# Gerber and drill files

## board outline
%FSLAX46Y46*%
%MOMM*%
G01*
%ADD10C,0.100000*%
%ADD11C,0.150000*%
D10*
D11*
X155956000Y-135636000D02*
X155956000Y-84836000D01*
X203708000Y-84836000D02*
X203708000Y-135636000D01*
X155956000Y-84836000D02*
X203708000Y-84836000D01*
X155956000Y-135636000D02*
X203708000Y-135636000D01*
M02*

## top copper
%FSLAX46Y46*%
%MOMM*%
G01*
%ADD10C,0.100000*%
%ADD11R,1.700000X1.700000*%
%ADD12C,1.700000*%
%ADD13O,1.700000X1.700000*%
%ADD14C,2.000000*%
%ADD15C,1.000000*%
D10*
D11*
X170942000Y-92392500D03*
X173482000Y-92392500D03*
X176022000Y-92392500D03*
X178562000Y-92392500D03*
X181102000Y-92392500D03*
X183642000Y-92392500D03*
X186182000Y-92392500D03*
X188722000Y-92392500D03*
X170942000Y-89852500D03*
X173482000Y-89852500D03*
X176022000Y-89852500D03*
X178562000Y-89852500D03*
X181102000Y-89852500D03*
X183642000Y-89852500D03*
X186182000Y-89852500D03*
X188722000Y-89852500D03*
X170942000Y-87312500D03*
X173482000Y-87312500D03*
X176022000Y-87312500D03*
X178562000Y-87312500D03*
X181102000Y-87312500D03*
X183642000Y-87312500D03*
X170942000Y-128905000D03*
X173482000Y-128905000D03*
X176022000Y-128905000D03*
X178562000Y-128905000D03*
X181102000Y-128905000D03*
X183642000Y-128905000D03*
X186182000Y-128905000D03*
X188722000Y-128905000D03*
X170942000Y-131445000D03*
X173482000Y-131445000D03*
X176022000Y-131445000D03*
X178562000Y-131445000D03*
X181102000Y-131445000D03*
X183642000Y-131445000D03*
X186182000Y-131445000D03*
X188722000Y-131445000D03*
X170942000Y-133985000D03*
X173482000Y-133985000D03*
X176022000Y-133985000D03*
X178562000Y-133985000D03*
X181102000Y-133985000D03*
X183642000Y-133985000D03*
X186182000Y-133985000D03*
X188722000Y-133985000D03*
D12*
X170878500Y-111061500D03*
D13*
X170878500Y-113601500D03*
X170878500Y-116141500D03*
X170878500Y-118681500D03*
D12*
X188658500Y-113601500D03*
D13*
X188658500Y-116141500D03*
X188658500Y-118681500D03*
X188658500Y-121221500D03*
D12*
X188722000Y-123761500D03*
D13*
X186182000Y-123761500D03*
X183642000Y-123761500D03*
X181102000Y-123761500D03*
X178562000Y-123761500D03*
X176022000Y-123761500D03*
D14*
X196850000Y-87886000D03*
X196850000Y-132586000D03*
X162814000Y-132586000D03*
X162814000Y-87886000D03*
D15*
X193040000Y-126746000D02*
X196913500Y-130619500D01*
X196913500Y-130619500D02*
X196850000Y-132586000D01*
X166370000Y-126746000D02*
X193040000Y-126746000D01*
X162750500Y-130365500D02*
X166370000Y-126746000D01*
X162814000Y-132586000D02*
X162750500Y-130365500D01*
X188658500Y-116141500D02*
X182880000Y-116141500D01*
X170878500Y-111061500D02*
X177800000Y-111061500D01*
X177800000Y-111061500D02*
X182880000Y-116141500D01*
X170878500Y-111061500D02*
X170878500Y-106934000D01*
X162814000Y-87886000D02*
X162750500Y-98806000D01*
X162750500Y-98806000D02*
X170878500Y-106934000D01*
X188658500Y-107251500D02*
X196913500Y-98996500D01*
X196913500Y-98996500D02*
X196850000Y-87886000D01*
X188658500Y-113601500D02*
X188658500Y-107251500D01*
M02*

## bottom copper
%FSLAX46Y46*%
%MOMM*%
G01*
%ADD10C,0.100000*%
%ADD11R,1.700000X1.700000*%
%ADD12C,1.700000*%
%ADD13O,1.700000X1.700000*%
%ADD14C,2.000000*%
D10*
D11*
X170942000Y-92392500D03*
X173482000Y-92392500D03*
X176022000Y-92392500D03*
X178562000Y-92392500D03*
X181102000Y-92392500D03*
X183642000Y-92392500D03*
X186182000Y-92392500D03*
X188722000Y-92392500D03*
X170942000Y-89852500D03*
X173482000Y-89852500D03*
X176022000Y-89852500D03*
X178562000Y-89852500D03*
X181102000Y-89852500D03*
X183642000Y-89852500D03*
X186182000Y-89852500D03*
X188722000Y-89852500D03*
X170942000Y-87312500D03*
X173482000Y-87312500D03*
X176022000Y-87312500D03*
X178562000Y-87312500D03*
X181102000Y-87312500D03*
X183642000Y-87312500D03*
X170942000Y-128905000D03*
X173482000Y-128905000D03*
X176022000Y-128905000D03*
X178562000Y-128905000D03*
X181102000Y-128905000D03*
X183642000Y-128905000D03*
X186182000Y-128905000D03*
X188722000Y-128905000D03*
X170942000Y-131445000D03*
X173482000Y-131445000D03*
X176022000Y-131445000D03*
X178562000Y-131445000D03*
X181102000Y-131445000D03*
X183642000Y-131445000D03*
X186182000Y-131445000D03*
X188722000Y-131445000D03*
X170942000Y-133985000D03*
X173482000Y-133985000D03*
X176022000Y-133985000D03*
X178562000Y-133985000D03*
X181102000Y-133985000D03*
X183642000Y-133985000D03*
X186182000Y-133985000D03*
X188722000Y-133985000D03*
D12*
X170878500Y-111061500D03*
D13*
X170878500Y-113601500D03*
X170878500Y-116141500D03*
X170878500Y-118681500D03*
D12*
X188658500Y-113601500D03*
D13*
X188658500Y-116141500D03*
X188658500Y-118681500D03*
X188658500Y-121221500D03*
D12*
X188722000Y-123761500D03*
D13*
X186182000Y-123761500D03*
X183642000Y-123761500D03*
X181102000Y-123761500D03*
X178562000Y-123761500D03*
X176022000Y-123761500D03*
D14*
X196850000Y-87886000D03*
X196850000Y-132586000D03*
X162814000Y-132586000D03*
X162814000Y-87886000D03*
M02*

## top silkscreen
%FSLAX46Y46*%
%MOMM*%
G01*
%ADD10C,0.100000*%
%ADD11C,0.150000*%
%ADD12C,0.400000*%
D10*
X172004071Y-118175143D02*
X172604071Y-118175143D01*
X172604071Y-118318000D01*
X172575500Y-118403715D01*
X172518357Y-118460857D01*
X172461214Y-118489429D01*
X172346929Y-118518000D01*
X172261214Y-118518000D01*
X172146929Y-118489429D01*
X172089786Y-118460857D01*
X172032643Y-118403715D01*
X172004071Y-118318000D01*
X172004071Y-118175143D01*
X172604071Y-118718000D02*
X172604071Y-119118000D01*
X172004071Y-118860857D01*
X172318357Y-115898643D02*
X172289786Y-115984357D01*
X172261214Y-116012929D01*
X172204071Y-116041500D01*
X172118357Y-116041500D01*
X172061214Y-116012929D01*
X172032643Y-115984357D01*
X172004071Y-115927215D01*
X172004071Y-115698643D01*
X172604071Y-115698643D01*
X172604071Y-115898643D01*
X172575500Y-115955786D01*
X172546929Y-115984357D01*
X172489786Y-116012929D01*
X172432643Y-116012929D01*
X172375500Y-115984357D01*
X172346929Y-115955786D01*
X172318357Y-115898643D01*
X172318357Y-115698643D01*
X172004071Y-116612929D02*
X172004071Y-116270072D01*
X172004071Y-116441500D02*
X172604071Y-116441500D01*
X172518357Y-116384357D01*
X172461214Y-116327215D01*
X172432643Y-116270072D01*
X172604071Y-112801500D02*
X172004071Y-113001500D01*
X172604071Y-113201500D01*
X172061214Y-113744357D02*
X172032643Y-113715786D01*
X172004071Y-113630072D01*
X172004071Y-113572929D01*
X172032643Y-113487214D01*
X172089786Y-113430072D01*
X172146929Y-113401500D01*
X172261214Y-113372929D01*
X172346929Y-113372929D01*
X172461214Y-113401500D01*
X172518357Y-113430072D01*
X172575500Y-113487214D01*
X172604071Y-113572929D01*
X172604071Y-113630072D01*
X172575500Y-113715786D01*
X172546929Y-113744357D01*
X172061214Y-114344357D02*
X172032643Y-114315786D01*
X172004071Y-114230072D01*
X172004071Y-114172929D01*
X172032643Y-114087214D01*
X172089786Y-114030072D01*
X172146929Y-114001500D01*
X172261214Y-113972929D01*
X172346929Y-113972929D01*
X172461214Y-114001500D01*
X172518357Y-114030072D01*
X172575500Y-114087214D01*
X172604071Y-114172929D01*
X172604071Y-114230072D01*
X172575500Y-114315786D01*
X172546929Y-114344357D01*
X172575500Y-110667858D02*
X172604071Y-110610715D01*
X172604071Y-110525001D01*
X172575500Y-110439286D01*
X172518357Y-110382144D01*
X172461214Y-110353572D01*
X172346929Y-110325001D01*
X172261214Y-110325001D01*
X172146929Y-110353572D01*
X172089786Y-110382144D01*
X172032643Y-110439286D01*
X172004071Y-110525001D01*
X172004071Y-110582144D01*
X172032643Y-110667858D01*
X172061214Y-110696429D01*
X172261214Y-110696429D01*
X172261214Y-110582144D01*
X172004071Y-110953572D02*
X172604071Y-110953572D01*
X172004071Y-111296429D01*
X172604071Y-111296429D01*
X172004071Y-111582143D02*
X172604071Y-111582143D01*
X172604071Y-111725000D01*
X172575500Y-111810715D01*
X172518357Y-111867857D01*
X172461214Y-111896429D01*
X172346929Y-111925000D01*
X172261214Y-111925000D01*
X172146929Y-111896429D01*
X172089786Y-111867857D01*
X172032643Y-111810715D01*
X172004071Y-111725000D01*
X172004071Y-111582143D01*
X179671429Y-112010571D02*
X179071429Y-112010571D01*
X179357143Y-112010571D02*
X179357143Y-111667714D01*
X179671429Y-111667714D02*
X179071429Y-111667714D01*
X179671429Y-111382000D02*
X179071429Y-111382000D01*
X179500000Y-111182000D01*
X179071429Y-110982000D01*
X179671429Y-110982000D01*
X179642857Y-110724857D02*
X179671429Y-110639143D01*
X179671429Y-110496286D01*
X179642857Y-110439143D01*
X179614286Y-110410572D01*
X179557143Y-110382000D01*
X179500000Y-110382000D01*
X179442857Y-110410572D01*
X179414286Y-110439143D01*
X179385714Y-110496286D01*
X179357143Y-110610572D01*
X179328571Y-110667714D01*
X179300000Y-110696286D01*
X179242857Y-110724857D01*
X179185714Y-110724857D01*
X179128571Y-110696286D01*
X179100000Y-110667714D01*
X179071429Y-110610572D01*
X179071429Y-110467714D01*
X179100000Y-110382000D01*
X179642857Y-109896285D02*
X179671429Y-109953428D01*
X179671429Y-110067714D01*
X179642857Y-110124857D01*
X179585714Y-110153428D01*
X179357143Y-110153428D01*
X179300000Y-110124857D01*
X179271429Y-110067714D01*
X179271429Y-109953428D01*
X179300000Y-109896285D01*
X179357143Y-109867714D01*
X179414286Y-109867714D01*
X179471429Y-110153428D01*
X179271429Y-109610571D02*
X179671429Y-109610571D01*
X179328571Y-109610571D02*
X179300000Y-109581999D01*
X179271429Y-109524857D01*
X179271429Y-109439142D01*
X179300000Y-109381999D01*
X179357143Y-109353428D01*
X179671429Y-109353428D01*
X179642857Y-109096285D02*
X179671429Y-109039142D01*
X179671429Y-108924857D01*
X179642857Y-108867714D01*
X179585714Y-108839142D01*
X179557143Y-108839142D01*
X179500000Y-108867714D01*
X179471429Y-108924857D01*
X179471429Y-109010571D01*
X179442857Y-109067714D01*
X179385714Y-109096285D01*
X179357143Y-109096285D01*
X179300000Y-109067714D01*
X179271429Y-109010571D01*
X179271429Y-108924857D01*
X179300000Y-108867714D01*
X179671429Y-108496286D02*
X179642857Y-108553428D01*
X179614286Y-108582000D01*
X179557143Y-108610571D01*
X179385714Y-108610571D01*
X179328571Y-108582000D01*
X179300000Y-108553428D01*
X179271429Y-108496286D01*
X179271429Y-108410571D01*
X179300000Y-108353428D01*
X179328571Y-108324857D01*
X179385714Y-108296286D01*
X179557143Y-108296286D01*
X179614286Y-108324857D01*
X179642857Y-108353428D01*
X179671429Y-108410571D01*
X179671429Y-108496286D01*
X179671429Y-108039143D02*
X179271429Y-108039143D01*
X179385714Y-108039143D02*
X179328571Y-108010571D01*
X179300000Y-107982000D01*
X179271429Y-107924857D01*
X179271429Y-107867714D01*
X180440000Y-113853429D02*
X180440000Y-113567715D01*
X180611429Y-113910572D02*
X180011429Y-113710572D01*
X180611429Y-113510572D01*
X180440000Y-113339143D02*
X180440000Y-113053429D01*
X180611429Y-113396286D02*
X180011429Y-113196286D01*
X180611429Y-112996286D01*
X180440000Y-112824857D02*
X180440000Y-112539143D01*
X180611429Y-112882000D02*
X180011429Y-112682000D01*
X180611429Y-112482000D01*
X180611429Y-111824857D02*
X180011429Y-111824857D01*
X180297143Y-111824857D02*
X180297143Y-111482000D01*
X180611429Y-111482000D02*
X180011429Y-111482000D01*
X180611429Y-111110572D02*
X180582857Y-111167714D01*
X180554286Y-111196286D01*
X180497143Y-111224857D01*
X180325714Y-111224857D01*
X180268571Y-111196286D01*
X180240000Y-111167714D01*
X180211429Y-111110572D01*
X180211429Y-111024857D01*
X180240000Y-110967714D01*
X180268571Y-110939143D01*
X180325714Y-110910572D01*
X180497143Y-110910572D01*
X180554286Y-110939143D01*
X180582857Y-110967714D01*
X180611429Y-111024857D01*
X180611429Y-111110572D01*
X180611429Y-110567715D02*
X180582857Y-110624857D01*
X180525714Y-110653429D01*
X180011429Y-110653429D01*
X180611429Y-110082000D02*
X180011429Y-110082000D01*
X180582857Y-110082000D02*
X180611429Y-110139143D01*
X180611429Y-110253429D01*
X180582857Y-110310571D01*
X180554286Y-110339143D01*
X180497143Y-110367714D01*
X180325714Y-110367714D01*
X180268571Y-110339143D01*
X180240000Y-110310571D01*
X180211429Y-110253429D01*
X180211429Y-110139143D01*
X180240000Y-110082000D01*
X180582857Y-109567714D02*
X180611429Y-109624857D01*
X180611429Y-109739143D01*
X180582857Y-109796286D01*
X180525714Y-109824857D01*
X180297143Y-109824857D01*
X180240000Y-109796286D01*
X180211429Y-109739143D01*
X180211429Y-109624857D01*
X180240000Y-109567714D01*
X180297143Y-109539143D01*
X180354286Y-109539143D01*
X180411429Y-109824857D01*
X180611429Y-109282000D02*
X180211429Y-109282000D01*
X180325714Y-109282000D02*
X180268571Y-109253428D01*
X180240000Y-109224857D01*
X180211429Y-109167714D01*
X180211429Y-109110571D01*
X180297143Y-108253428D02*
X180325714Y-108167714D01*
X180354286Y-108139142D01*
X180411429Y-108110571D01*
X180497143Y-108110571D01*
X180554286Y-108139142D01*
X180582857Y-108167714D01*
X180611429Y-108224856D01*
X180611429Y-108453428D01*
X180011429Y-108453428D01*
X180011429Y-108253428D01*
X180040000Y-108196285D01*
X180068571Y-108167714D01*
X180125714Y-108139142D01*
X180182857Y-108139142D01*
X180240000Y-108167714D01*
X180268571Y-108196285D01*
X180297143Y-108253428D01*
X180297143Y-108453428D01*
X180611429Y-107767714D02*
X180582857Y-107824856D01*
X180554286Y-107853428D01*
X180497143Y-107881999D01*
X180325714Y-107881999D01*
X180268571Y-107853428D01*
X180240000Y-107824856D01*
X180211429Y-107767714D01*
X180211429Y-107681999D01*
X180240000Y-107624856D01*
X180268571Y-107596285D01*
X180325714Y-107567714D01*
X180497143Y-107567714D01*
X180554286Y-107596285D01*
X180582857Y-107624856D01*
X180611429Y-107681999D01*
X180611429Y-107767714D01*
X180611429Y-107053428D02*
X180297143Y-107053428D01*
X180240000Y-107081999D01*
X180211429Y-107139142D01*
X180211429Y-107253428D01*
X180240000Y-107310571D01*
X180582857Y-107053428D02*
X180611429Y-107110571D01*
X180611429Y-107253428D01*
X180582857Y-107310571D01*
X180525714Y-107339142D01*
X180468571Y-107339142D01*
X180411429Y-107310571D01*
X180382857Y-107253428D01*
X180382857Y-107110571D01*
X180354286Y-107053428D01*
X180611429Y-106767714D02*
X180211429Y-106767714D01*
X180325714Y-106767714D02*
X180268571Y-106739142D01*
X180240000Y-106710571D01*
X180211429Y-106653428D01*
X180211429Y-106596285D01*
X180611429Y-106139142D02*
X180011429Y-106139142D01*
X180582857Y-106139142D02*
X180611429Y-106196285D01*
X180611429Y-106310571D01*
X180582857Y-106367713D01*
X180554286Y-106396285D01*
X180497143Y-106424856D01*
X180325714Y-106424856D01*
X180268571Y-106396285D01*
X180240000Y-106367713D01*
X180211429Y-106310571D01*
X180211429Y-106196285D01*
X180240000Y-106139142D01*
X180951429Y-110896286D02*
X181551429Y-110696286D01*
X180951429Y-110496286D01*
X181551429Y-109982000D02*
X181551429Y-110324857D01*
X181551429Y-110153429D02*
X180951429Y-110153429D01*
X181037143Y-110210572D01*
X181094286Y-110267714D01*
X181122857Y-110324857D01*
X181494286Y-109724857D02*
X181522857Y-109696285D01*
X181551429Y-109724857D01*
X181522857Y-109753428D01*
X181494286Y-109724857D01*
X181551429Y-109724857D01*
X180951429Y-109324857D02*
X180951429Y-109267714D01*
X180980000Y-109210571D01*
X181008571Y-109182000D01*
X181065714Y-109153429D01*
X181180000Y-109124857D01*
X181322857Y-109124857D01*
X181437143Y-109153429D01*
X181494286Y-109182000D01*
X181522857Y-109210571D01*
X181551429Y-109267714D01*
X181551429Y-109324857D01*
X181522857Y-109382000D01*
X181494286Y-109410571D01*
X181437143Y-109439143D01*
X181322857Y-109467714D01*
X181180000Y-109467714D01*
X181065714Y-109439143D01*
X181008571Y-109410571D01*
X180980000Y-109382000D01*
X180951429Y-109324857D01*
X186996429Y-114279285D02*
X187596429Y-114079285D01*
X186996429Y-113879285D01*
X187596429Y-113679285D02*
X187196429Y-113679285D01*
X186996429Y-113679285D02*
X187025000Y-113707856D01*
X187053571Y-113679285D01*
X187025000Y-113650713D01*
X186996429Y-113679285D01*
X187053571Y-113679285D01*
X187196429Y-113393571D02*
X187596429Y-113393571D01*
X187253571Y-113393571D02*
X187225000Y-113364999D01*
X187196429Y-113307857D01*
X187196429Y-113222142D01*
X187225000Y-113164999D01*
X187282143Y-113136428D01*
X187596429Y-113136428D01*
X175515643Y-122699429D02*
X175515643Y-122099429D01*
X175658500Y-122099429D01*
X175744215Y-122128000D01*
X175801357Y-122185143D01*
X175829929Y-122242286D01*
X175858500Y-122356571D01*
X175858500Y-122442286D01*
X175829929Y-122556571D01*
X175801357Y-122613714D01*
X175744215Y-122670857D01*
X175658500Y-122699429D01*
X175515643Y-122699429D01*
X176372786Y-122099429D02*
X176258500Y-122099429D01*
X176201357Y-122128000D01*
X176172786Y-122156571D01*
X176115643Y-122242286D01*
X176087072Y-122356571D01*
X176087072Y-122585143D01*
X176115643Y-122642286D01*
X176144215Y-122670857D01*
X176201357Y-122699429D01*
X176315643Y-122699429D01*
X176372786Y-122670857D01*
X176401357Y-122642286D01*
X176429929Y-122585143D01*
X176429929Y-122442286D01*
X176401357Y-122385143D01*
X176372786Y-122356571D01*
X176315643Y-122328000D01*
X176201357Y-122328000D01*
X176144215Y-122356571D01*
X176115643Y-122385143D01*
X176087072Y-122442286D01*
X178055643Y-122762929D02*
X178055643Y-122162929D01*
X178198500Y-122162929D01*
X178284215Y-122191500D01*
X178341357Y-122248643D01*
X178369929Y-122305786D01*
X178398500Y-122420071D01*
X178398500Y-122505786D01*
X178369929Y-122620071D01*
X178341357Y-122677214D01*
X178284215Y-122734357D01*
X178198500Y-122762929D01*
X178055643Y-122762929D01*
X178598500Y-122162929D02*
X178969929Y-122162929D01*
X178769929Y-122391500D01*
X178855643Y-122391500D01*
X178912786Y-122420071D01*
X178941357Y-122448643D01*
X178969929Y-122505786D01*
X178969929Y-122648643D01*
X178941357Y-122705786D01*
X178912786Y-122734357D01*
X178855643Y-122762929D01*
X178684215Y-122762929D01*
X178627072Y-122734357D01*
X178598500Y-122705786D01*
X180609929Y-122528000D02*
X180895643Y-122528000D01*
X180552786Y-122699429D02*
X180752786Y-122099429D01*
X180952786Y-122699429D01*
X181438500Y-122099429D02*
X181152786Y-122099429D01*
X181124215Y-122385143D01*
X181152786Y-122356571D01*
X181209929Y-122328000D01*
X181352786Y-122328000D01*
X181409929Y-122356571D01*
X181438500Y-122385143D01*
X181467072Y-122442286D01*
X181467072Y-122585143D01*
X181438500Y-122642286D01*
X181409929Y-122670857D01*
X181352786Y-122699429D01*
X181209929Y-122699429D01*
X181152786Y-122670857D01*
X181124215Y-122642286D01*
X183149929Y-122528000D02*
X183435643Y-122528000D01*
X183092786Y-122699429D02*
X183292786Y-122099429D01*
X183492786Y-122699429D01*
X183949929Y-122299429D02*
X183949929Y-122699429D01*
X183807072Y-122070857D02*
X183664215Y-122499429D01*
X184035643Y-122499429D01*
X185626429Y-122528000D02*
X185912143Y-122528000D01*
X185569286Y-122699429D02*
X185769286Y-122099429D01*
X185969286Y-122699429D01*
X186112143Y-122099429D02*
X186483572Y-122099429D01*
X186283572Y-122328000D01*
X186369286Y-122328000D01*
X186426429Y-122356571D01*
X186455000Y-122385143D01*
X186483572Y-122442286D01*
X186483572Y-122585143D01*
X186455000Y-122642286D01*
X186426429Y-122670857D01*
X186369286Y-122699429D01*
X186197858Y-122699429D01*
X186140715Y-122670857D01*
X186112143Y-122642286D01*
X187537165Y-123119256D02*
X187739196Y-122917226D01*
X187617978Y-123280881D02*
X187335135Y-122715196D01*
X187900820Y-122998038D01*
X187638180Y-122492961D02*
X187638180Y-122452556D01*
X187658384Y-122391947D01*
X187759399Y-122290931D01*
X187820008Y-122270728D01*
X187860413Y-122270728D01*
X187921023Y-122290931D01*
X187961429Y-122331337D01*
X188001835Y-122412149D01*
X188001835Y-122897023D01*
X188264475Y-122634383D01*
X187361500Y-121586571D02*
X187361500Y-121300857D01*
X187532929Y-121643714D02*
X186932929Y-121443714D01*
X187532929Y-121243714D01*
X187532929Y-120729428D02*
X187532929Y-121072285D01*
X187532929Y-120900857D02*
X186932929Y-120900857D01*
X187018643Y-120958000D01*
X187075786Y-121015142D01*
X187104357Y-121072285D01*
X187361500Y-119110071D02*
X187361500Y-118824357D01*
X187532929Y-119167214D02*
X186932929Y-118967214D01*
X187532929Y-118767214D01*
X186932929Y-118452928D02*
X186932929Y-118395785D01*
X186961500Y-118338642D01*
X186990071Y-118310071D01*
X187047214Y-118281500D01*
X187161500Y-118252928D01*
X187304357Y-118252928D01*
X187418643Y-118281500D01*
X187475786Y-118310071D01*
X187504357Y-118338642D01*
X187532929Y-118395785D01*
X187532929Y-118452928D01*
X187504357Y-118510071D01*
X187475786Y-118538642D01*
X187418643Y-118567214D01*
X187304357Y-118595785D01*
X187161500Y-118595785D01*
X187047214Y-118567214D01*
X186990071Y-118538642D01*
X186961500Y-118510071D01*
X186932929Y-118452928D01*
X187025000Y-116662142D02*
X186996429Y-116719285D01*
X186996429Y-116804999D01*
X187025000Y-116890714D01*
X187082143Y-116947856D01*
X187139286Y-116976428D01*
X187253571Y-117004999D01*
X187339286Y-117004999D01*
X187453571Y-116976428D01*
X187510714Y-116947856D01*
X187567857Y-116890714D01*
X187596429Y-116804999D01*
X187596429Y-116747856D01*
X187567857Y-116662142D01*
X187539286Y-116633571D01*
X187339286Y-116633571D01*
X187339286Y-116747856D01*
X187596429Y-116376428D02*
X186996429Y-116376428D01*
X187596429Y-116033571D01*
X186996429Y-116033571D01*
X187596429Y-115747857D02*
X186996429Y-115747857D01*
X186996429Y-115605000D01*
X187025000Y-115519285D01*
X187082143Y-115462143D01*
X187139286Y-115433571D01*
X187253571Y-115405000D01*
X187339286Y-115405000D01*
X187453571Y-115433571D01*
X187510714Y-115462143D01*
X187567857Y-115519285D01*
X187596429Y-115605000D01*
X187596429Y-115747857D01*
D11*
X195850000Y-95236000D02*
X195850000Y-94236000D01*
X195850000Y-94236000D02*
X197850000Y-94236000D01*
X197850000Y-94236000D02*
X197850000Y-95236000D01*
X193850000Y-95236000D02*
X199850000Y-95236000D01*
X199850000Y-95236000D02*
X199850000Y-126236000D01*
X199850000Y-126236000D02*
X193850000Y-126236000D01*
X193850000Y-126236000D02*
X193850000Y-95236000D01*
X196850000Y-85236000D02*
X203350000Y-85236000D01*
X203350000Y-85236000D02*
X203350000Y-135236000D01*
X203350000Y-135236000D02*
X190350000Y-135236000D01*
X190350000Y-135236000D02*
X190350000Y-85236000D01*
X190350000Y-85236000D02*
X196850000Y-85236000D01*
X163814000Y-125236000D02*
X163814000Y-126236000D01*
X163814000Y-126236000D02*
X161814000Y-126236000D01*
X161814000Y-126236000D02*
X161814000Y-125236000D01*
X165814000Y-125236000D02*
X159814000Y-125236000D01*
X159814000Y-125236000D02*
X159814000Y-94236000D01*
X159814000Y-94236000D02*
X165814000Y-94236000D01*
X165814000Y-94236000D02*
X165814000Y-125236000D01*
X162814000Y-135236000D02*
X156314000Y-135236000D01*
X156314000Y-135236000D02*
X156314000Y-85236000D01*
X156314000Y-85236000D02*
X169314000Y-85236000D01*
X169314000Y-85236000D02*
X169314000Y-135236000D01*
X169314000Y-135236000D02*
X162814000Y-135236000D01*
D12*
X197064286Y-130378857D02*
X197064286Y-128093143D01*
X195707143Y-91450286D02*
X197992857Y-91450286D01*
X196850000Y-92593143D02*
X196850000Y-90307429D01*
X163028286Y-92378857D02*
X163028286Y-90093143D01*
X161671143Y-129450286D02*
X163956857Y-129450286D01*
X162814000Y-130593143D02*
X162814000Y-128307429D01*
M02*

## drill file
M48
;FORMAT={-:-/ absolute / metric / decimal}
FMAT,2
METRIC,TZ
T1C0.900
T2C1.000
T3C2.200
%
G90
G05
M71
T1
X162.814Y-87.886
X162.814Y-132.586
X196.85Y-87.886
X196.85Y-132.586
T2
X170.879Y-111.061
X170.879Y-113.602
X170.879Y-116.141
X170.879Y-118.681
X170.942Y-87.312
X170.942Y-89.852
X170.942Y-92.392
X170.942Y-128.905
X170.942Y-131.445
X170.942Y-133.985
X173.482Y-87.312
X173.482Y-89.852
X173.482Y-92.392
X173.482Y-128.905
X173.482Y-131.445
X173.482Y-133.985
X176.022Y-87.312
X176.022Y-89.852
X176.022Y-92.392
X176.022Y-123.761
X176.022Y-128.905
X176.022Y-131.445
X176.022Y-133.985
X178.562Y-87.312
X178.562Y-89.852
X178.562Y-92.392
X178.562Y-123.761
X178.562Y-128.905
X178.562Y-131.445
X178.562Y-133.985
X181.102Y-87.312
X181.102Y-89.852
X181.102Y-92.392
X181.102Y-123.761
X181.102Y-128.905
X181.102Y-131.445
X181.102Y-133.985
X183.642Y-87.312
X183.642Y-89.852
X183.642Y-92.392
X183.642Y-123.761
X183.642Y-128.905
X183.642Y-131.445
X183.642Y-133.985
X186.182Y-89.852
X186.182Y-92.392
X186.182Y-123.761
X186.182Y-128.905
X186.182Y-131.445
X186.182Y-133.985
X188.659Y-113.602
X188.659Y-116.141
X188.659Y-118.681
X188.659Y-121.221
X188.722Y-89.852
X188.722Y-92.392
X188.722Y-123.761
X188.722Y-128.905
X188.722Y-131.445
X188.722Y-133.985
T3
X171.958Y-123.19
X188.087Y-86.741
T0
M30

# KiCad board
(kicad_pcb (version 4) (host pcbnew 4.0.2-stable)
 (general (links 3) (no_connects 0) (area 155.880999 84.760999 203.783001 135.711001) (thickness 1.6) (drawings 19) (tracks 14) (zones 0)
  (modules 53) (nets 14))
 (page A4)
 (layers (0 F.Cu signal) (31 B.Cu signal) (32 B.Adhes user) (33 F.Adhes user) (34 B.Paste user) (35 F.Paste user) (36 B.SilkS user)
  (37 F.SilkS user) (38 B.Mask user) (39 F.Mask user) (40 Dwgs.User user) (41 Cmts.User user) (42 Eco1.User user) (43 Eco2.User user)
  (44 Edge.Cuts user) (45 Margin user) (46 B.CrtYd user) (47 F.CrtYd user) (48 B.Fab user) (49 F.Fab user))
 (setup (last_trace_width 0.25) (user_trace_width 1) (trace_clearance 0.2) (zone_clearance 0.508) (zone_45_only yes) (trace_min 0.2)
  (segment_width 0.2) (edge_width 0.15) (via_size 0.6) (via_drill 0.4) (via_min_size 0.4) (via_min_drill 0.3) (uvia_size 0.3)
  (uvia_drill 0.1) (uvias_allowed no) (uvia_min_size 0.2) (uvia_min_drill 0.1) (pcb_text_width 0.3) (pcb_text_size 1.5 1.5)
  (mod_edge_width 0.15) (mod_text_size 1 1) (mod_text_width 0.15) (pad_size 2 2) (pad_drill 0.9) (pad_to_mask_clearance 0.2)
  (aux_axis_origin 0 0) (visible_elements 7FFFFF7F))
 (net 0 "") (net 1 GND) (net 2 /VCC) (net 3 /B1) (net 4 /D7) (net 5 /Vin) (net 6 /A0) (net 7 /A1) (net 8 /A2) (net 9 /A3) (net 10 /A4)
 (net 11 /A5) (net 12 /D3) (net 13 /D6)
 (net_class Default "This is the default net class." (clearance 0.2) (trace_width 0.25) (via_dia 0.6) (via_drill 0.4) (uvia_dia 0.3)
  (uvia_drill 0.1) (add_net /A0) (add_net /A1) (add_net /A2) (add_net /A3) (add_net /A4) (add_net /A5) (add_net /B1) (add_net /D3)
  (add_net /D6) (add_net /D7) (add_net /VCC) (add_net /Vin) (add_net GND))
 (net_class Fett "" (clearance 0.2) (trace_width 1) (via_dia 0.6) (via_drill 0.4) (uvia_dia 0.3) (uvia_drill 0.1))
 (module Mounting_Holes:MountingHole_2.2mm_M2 (layer F.Cu) (at 188.087 86.741)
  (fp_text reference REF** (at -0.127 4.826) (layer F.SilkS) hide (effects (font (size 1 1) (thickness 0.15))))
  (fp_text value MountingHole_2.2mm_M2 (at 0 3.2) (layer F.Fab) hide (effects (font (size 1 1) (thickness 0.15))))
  (pad 1 np_thru_hole circle (at 0 0) (size 2.2 2.2) (drill 2.2) (layers *.Cu *.Mask)))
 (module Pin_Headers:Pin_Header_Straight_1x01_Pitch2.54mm (layer F.Cu) (at 170.942 92.3925)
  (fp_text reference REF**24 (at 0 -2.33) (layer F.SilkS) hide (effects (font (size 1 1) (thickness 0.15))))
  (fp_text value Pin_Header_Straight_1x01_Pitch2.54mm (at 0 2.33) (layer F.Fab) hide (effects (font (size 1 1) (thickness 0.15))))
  (pad 1 thru_hole rect (at 0 0) (size 1.7 1.7) (drill 1) (layers *.Cu *.Mask)))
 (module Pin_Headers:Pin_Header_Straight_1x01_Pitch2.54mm (layer F.Cu) (at 173.482 92.3925)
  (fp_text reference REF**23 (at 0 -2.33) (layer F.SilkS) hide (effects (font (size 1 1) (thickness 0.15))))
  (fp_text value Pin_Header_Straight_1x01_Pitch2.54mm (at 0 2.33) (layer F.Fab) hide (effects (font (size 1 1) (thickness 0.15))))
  (pad 1 thru_hole rect (at 0 0) (size 1.7 1.7) (drill 1) (layers *.Cu *.Mask)))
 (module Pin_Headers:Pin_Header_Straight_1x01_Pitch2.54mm (layer F.Cu) (at 176.022 92.3925)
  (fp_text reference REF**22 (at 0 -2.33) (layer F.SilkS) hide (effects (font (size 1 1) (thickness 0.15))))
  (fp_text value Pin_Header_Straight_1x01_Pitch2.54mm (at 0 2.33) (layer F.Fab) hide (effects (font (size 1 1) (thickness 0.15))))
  (pad 1 thru_hole rect (at 0 0) (size 1.7 1.7) (drill 1) (layers *.Cu *.Mask)))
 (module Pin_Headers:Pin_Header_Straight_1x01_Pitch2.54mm (layer F.Cu) (at 178.562 92.3925)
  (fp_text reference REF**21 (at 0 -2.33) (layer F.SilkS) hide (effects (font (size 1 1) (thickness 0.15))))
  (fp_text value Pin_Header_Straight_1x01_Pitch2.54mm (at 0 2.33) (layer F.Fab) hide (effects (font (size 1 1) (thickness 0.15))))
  (pad 1 thru_hole rect (at 0 0) (size 1.7 1.7) (drill 1) (layers *.Cu *.Mask)))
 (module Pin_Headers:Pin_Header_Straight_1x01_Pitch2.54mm (layer F.Cu) (at 181.102 92.3925)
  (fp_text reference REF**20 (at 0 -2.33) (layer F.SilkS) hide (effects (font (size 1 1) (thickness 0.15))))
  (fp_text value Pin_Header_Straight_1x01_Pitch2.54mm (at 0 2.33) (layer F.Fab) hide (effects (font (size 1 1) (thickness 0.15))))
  (pad 1 thru_hole rect (at 0 0) (size 1.7 1.7) (drill 1) (layers *.Cu *.Mask)))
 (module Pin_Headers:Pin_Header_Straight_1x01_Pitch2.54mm (layer F.Cu) (at 183.642 92.3925)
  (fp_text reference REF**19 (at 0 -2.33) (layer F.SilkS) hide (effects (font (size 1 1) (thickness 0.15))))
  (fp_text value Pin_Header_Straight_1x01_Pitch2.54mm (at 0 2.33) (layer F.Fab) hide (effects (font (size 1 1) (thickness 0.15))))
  (pad 1 thru_hole rect (at 0 0) (size 1.7 1.7) (drill 1) (layers *.Cu *.Mask)))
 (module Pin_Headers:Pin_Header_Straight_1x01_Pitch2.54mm (layer F.Cu) (at 186.182 92.3925)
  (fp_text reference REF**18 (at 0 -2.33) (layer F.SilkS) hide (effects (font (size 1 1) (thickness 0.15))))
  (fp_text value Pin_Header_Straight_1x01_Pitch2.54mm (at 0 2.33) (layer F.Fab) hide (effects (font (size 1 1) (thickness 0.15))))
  (pad 1 thru_hole rect (at 0 0) (size 1.7 1.7) (drill 1) (layers *.Cu *.Mask)))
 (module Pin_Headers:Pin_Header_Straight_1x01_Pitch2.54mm (layer F.Cu) (at 188.722 92.3925)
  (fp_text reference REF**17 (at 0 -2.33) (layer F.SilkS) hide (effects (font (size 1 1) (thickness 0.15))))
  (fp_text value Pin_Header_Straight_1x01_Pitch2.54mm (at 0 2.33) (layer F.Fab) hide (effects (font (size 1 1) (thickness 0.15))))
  (pad 1 thru_hole rect (at 0 0) (size 1.7 1.7) (drill 1) (layers *.Cu *.Mask)))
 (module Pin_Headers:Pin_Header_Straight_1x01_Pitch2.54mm (layer F.Cu) (at 170.942 89.8525)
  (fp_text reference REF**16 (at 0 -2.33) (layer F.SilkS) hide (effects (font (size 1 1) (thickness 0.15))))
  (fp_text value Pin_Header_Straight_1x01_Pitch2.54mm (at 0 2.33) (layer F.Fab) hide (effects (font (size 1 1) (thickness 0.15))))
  (pad 1 thru_hole rect (at 0 0) (size 1.7 1.7) (drill 1) (layers *.Cu *.Mask)))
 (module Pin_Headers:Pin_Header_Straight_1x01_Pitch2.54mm (layer F.Cu) (at 173.482 89.8525)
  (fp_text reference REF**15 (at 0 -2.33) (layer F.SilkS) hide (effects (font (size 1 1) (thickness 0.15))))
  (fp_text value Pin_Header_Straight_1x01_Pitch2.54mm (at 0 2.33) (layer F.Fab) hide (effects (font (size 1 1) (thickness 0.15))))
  (pad 1 thru_hole rect (at 0 0) (size 1.7 1.7) (drill 1) (layers *.Cu *.Mask)))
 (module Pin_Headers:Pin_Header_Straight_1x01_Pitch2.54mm (layer F.Cu) (at 176.022 89.8525)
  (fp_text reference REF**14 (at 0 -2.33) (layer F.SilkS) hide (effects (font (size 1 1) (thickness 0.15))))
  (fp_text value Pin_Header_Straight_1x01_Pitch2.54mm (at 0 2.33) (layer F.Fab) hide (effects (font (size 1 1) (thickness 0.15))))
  (pad 1 thru_hole rect (at 0 0) (size 1.7 1.7) (drill 1) (layers *.Cu *.Mask)))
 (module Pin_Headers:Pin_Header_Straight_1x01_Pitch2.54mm (layer F.Cu) (at 178.562 89.8525)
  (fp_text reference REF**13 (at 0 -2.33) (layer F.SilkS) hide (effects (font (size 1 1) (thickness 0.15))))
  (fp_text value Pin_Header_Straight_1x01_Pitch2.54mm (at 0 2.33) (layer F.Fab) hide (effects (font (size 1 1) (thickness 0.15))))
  (pad 1 thru_hole rect (at 0 0) (size 1.7 1.7) (drill 1) (layers *.Cu *.Mask)))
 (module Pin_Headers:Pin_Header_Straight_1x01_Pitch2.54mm (layer F.Cu) (at 181.102 89.8525)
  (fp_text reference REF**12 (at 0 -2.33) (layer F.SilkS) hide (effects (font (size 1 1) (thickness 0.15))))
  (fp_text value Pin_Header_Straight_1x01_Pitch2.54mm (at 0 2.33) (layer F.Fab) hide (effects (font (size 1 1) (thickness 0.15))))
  (pad 1 thru_hole rect (at 0 0) (size 1.7 1.7) (drill 1) (layers *.Cu *.Mask)))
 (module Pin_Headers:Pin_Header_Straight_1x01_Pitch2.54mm (layer F.Cu) (at 183.642 89.8525)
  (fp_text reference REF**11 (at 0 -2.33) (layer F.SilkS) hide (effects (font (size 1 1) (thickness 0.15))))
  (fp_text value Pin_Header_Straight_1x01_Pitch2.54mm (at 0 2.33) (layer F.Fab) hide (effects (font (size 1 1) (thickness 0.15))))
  (pad 1 thru_hole rect (at 0 0) (size 1.7 1.7) (drill 1) (layers *.Cu *.Mask)))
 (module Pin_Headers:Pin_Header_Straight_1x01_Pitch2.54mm (layer F.Cu) (at 186.182 89.8525)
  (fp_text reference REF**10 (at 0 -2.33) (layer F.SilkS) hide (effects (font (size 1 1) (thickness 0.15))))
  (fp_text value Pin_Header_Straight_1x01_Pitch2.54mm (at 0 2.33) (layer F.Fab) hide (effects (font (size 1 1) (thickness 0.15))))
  (pad 1 thru_hole rect (at 0 0) (size 1.7 1.7) (drill 1) (layers *.Cu *.Mask)))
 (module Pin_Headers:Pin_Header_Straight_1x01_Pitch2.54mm (layer F.Cu) (at 188.722 89.8525)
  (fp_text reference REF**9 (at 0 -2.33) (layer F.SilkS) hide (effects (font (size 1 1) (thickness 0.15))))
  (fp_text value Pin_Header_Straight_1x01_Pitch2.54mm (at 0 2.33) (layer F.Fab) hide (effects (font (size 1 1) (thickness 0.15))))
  (pad 1 thru_hole rect (at 0 0) (size 1.7 1.7) (drill 1) (layers *.Cu *.Mask)))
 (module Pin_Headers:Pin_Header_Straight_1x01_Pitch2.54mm (layer F.Cu) (at 170.942 87.3125)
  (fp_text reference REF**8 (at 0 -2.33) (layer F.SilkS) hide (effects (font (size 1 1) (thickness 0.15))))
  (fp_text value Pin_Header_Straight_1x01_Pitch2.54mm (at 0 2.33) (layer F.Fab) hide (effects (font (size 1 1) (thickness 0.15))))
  (pad 1 thru_hole rect (at 0 0) (size 1.7 1.7) (drill 1) (layers *.Cu *.Mask)))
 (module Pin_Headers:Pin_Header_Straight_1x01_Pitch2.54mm (layer F.Cu) (at 173.482 87.3125)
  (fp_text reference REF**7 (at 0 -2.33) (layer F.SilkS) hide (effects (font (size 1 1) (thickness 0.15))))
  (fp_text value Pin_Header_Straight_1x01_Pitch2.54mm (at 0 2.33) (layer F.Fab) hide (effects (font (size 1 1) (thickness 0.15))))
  (pad 1 thru_hole rect (at 0 0) (size 1.7 1.7) (drill 1) (layers *.Cu *.Mask)))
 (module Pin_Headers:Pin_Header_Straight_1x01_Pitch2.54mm (layer F.Cu) (at 176.022 87.3125)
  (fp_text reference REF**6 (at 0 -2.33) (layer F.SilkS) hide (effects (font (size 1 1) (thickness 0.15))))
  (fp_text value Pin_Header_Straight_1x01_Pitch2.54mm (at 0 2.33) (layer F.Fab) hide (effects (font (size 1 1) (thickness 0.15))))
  (pad 1 thru_hole rect (at 0 0) (size 1.7 1.7) (drill 1) (layers *.Cu *.Mask)))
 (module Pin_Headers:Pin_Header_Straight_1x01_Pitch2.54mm (layer F.Cu) (at 178.562 87.3125)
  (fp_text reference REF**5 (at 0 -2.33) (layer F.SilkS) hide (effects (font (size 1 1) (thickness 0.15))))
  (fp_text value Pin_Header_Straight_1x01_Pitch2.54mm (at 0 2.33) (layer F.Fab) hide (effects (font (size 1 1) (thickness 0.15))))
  (pad 1 thru_hole rect (at 0 0) (size 1.7 1.7) (drill 1) (layers *.Cu *.Mask)))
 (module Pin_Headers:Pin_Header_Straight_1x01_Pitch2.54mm (layer F.Cu) (at 181.102 87.3125)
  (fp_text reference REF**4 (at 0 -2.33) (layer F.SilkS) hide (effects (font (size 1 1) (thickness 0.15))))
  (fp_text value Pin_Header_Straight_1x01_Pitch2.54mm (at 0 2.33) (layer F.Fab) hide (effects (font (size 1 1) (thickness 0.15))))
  (pad 1 thru_hole rect (at 0 0) (size 1.7 1.7) (drill 1) (layers *.Cu *.Mask)))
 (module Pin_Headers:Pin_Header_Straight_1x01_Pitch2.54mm (layer F.Cu) (at 183.642 87.3125)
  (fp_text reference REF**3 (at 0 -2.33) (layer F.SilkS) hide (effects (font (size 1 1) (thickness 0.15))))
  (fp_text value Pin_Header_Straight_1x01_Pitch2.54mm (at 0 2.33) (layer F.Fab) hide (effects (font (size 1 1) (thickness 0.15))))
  (pad 1 thru_hole rect (at 0 0) (size 1.7 1.7) (drill 1) (layers *.Cu *.Mask)))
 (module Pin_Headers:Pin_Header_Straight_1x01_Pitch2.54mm (layer F.Cu) (at 170.942 128.905)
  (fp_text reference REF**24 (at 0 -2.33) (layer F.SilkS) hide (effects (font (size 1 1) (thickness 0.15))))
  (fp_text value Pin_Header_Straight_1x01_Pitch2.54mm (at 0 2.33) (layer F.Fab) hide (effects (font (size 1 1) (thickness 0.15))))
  (pad 1 thru_hole rect (at 0 0) (size 1.7 1.7) (drill 1) (layers *.Cu *.Mask)))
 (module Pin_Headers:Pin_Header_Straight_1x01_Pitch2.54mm (layer F.Cu) (at 173.482 128.905)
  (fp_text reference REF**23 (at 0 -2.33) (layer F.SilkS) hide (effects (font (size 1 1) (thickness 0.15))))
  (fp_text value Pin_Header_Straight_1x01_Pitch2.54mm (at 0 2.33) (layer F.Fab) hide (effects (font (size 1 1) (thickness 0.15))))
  (pad 1 thru_hole rect (at 0 0) (size 1.7 1.7) (drill 1) (layers *.Cu *.Mask)))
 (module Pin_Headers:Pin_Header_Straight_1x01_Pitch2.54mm (layer F.Cu) (at 176.022 128.905)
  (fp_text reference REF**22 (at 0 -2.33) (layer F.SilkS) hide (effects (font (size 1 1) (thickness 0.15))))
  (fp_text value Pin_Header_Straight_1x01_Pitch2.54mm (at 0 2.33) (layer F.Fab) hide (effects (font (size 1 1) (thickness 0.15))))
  (pad 1 thru_hole rect (at 0 0) (size 1.7 1.7) (drill 1) (layers *.Cu *.Mask)))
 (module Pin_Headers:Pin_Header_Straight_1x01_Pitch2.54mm (layer F.Cu) (at 178.562 128.905)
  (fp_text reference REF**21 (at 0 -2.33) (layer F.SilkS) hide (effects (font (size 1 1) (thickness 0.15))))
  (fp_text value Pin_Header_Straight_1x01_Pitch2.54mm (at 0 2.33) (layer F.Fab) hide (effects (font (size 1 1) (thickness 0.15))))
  (pad 1 thru_hole rect (at 0 0) (size 1.7 1.7) (drill 1) (layers *.Cu *.Mask)))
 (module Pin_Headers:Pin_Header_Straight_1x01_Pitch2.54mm (layer F.Cu) (at 181.102 128.905)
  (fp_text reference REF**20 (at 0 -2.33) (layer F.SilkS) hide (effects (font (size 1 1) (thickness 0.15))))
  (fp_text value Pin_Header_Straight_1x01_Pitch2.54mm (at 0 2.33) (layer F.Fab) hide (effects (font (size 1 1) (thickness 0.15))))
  (pad 1 thru_hole rect (at 0 0) (size 1.7 1.7) (drill 1) (layers *.Cu *.Mask)))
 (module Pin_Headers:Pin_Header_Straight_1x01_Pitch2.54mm (layer F.Cu) (at 183.642 128.905)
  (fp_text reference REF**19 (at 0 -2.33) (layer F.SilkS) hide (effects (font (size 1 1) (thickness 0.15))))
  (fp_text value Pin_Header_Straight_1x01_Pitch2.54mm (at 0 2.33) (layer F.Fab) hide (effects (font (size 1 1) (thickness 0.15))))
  (pad 1 thru_hole rect (at 0 0) (size 1.7 1.7) (drill 1) (layers *.Cu *.Mask)))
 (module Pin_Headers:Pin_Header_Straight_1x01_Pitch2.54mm (layer F.Cu) (at 186.182 128.905)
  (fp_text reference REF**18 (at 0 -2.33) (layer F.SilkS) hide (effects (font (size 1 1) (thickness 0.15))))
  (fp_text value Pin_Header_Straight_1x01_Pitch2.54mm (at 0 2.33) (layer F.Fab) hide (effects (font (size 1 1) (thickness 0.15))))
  (pad 1 thru_hole rect (at 0 0) (size 1.7 1.7) (drill 1) (layers *.Cu *.Mask)))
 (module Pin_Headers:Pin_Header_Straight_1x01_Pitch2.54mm (layer F.Cu) (at 188.722 128.905)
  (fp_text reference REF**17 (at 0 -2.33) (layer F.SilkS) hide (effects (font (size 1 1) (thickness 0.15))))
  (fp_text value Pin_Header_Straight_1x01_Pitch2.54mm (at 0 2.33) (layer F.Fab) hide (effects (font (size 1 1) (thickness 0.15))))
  (pad 1 thru_hole rect (at 0 0) (size 1.7 1.7) (drill 1) (layers *.Cu *.Mask)))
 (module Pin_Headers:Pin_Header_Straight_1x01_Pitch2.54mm (layer F.Cu) (at 170.942 131.445)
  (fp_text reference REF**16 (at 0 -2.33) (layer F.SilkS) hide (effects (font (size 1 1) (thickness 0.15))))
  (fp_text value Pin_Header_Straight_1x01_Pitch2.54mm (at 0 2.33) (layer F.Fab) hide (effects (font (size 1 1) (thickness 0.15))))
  (pad 1 thru_hole rect (at 0 0) (size 1.7 1.7) (drill 1) (layers *.Cu *.Mask)))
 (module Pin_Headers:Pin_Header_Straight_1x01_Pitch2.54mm (layer F.Cu) (at 173.482 131.445)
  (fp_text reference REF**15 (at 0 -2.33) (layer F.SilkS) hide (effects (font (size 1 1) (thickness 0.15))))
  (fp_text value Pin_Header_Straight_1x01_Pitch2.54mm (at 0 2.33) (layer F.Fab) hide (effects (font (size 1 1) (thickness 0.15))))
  (pad 1 thru_hole rect (at 0 0) (size 1.7 1.7) (drill 1) (layers *.Cu *.Mask)))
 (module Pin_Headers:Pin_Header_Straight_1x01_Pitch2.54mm (layer F.Cu) (at 176.022 131.445)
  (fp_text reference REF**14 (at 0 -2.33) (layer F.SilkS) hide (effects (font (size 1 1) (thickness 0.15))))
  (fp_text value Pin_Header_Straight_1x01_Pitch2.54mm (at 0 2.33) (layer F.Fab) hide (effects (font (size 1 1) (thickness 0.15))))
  (pad 1 thru_hole rect (at 0 0) (size 1.7 1.7) (drill 1) (layers *.Cu *.Mask)))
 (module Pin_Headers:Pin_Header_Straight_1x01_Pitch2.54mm (layer F.Cu) (at 178.562 131.445)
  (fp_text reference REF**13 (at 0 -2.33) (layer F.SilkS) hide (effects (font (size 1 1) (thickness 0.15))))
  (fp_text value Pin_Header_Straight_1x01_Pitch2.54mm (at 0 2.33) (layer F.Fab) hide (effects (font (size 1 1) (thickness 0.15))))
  (pad 1 thru_hole rect (at 0 0) (size 1.7 1.7) (drill 1) (layers *.Cu *.Mask)))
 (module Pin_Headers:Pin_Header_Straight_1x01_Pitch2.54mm (layer F.Cu) (at 181.102 131.445)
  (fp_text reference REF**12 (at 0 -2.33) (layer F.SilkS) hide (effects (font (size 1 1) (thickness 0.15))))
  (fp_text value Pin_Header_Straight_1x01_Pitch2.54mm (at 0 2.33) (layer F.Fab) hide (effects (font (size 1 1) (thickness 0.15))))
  (pad 1 thru_hole rect (at 0 0) (size 1.7 1.7) (drill 1) (layers *.Cu *.Mask)))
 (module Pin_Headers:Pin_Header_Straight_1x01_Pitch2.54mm (layer F.Cu) (at 183.642 131.445)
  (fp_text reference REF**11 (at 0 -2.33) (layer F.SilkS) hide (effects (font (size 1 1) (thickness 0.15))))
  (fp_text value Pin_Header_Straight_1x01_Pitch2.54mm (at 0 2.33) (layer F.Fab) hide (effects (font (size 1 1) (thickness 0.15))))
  (pad 1 thru_hole rect (at 0 0) (size 1.7 1.7) (drill 1) (layers *.Cu *.Mask)))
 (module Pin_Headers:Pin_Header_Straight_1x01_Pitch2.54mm (layer F.Cu) (at 186.182 131.445)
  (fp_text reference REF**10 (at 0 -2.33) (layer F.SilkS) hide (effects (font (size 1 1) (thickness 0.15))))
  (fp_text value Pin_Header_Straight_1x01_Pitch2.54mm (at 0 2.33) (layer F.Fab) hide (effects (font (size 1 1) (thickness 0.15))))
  (pad 1 thru_hole rect (at 0 0) (size 1.7 1.7) (drill 1) (layers *.Cu *.Mask)))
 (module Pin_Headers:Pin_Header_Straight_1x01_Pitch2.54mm (layer F.Cu) (at 188.722 131.445)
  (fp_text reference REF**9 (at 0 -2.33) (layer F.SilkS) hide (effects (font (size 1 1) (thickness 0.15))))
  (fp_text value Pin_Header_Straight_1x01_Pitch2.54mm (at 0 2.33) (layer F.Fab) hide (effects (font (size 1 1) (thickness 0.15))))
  (pad 1 thru_hole rect (at 0 0) (size 1.7 1.7) (drill 1) (layers *.Cu *.Mask)))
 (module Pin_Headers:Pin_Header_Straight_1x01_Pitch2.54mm (layer F.Cu) (at 170.942 133.985)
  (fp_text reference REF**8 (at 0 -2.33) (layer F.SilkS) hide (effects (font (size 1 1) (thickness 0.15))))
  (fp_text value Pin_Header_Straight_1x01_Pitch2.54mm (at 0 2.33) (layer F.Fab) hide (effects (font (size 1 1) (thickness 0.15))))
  (pad 1 thru_hole rect (at 0 0) (size 1.7 1.7) (drill 1) (layers *.Cu *.Mask)))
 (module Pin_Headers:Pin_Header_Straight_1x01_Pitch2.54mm (layer F.Cu) (at 173.482 133.985)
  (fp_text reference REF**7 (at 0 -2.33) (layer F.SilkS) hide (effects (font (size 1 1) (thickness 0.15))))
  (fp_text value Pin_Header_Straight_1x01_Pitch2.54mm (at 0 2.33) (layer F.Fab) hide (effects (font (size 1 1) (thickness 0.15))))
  (pad 1 thru_hole rect (at 0 0) (size 1.7 1.7) (drill 1) (layers *.Cu *.Mask)))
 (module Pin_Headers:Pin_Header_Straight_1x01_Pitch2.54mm (layer F.Cu) (at 176.022 133.985)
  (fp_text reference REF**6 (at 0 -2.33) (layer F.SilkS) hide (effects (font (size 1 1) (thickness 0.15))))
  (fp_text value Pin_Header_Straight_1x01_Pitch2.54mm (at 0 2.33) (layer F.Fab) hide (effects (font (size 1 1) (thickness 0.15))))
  (pad 1 thru_hole rect (at 0 0) (size 1.7 1.7) (drill 1) (layers *.Cu *.Mask)))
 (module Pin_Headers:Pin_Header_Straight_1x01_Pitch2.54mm (layer F.Cu) (at 178.562 133.985)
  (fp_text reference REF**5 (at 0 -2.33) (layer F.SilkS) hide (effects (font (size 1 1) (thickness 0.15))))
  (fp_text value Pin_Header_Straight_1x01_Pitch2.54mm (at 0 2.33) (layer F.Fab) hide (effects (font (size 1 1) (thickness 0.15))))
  (pad 1 thru_hole rect (at 0 0) (size 1.7 1.7) (drill 1) (layers *.Cu *.Mask)))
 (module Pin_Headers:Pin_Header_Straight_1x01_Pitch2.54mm (layer F.Cu) (at 181.102 133.985)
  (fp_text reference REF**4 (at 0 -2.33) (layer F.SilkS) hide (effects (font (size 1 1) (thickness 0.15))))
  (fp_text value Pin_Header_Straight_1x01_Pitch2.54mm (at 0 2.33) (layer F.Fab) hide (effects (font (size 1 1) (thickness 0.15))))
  (pad 1 thru_hole rect (at 0 0) (size 1.7 1.7) (drill 1) (layers *.Cu *.Mask)))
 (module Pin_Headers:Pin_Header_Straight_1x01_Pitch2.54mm (layer F.Cu) (at 183.642 133.985)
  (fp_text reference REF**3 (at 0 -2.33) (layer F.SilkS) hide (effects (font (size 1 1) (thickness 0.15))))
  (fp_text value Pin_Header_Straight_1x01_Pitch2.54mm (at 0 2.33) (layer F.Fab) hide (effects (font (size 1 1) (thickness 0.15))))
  (pad 1 thru_hole rect (at 0 0) (size 1.7 1.7) (drill 1) (layers *.Cu *.Mask)))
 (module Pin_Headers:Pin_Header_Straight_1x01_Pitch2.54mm (layer F.Cu) (at 186.182 133.985)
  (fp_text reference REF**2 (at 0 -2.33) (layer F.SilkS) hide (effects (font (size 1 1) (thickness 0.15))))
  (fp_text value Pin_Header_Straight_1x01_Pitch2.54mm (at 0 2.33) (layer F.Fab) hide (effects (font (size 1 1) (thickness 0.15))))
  (pad 1 thru_hole rect (at 0 0) (size 1.7 1.7) (drill 1) (layers *.Cu *.Mask)))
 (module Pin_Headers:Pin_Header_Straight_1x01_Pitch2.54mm (layer F.Cu) (at 188.722 133.985)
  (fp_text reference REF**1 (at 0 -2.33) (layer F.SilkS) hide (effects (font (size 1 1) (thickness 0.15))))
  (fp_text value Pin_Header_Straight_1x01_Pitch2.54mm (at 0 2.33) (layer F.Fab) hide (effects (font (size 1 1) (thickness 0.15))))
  (pad 1 thru_hole rect (at 0 0) (size 1.7 1.7) (drill 1) (layers *.Cu *.Mask)))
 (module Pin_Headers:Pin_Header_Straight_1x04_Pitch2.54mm (layer F.Cu) (at 170.8785 111.0615)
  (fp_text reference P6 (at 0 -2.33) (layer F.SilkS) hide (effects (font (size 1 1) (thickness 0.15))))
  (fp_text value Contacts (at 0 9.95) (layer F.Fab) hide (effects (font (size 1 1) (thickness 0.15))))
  (pad 1 thru_hole circle (at 0 0) (size 1.7 1.7) (drill 1) (layers *.Cu *.Mask) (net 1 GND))
  (pad 2 thru_hole oval (at 0 2.54) (size 1.7 1.7) (drill 1) (layers *.Cu *.Mask) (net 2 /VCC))
  (pad 3 thru_hole oval (at 0 5.08) (size 1.7 1.7) (drill 1) (layers *.Cu *.Mask) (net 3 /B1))
  (pad 4 thru_hole oval (at 0 7.62) (size 1.7 1.7) (drill 1) (layers *.Cu *.Mask) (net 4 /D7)))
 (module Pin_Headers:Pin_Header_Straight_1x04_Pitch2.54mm (layer F.Cu) (at 188.6585 113.6015)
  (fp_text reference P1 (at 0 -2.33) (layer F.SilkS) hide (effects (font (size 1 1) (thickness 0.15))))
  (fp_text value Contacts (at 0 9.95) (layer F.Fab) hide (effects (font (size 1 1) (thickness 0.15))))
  (pad 1 thru_hole circle (at 0 0) (size 1.7 1.7) (drill 1) (layers *.Cu *.Mask) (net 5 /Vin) (zone_connect 2))
  (pad 2 thru_hole oval (at 0 2.54) (size 1.7 1.7) (drill 1) (layers *.Cu *.Mask) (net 1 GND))
  (pad 3 thru_hole oval (at 0 5.08) (size 1.7 1.7) (drill 1) (layers *.Cu *.Mask) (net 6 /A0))
  (pad 4 thru_hole oval (at 0 7.62) (size 1.7 1.7) (drill 1) (layers *.Cu *.Mask) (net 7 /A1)))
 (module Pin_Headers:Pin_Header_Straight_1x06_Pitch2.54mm (layer F.Cu) (at 188.722 123.7615 270)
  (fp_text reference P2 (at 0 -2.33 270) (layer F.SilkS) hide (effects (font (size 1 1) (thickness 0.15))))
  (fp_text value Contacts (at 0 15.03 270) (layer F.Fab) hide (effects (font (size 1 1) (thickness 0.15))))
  (pad 1 thru_hole circle (at 0 0 270) (size 1.7 1.7) (drill 1) (layers *.Cu *.Mask) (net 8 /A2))
  (pad 2 thru_hole oval (at 0 2.54 270) (size 1.7 1.7) (drill 1) (layers *.Cu *.Mask) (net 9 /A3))
  (pad 3 thru_hole oval (at 0 5.08 270) (size 1.7 1.7) (drill 1) (layers *.Cu *.Mask) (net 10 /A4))
  (pad 4 thru_hole oval (at 0 7.62 270) (size 1.7 1.7) (drill 1) (layers *.Cu *.Mask) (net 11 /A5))
  (pad 5 thru_hole oval (at 0 10.16 270) (size 1.7 1.7) (drill 1) (layers *.Cu *.Mask) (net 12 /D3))
  (pad 6 thru_hole oval (at 0 12.7 270) (size 1.7 1.7) (drill 1) (layers *.Cu *.Mask) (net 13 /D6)))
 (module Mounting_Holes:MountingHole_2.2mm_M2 (layer F.Cu) (at 171.958 123.19)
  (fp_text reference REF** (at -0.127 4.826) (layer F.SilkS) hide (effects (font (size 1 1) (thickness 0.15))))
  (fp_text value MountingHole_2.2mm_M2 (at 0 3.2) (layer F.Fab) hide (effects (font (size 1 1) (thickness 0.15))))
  (pad 1 np_thru_hole circle (at 0 0) (size 2.2 2.2) (drill 2.2) (layers *.Cu *.Mask)))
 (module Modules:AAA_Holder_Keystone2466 (layer F.Cu) (at 196.85 110.236)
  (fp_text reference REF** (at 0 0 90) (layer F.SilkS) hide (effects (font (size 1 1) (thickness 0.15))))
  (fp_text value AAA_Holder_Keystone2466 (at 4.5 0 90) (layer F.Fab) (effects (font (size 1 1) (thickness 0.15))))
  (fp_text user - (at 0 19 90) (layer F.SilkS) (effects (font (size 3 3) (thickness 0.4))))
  (fp_line (start -1 -15) (end -1 -16) (layer F.SilkS) (width 0.15))
  (fp_line (start -1 -16) (end 1 -16) (layer F.SilkS) (width 0.15))
  (fp_line (start 1 -16) (end 1 -15) (layer F.SilkS) (width 0.15))
  (fp_line (start -3 -15) (end 3 -15) (layer F.SilkS) (width 0.15))
  (fp_line (start 3 -15) (end 3 16) (layer F.SilkS) (width 0.15))
  (fp_line (start 3 16) (end -3 16) (layer F.SilkS) (width 0.15))
  (fp_line (start -3 16) (end -3 -15) (layer F.SilkS) (width 0.15))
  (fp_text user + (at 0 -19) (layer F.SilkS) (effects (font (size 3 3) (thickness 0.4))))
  (fp_line (start 0 -25) (end 6.5 -25) (layer F.SilkS) (width 0.15))
  (fp_line (start 6.5 -25) (end 6.5 25) (layer F.SilkS) (width 0.15))
  (fp_line (start 6.5 25) (end -6.5 25) (layer F.SilkS) (width 0.15))
  (fp_line (start -6.5 25) (end -6.5 -25) (layer F.SilkS) (width 0.15))
  (fp_line (start -6.5 -25) (end 0 -25) (layer F.SilkS) (width 0.15))
  (pad 1 thru_hole circle (at 0 -22.35) (size 2 2) (drill 0.9) (layers *.Cu *.Mask F.SilkS) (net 5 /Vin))
  (pad 2 thru_hole circle (at 0 22.35) (size 2 2) (drill 0.9) (layers *.Cu *.Mask F.SilkS)))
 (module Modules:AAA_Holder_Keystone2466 (layer F.Cu) (at 162.814 110.236 180)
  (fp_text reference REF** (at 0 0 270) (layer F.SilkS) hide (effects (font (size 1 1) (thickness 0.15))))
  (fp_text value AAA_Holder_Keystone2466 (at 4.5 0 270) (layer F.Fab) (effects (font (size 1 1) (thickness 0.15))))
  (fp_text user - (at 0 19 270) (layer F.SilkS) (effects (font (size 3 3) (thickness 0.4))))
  (fp_line (start -1 -15) (end -1 -16) (layer F.SilkS) (width 0.15))
  (fp_line (start -1 -16) (end 1 -16) (layer F.SilkS) (width 0.15))
  (fp_line (start 1 -16) (end 1 -15) (layer F.SilkS) (width 0.15))
  (fp_line (start -3 -15) (end 3 -15) (layer F.SilkS) (width 0.15))
  (fp_line (start 3 -15) (end 3 16) (layer F.SilkS) (width 0.15))
  (fp_line (start 3 16) (end -3 16) (layer F.SilkS) (width 0.15))
  (fp_line (start -3 16) (end -3 -15) (layer F.SilkS) (width 0.15))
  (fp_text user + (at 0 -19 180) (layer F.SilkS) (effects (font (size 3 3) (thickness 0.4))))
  (fp_line (start 0 -25) (end 6.5 -25) (layer F.SilkS) (width 0.15))
  (fp_line (start 6.5 -25) (end 6.5 25) (layer F.SilkS) (width 0.15))
  (fp_line (start 6.5 25) (end -6.5 25) (layer F.SilkS) (width 0.15))
  (fp_line (start -6.5 25) (end -6.5 -25) (layer F.SilkS) (width 0.15))
  (fp_line (start -6.5 -25) (end 0 -25) (layer F.SilkS) (width 0.15))
  (pad 1 thru_hole circle (at 0 -22.35 180) (size 2 2) (drill 0.9) (layers *.Cu *.Mask F.SilkS))
  (pad 2 thru_hole circle (at 0 22.35 180) (size 2 2) (drill 0.9) (layers *.Cu *.Mask F.SilkS) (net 1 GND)))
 (gr_line (start 155.956 135.636) (end 155.956 84.836) (angle 90) (layer Edge.Cuts) (width 0.15))
 (gr_line (start 203.708 84.836) (end 203.708 135.636) (angle 90) (layer Edge.Cuts) (width 0.15))
 (gr_line (start 155.956 84.836) (end 203.708 84.836) (angle 90) (layer Edge.Cuts) (width 0.15))
 (gr_line (start 155.956 135.636) (end 203.708 135.636) (angle 90) (layer Edge.Cuts) (width 0.15))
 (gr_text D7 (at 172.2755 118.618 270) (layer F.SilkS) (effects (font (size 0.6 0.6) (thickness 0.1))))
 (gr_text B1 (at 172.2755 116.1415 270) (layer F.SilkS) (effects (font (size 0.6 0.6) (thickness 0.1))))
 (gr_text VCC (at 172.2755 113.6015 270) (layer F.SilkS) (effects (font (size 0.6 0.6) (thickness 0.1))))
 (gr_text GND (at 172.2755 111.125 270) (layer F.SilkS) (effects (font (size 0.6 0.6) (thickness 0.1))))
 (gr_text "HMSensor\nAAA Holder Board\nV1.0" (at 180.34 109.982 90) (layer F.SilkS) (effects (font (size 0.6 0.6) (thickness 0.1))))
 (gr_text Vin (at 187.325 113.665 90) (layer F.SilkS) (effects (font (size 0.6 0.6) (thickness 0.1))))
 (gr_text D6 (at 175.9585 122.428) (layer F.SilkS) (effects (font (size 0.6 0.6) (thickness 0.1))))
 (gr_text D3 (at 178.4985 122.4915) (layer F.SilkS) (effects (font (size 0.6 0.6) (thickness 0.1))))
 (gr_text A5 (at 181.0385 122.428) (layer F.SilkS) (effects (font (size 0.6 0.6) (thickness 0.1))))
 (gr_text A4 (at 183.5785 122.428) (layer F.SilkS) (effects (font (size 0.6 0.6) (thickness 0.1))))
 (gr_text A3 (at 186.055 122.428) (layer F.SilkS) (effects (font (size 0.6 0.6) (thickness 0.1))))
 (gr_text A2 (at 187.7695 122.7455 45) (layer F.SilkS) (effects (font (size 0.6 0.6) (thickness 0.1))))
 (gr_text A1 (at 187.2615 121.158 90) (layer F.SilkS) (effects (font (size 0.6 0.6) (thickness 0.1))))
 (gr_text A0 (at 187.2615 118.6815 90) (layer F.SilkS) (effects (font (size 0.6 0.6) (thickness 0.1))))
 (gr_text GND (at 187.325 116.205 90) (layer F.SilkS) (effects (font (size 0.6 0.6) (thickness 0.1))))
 (segment (start 193.04 126.746) (end 196.9135 130.6195) (width 1) (layer F.Cu) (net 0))
 (segment (start 196.9135 130.6195) (end 196.85 132.586) (width 1) (layer F.Cu) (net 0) (status 20))
 (segment (start 166.37 126.746) (end 193.04 126.746) (width 1) (layer F.Cu) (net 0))
 (segment (start 162.7505 130.3655) (end 166.37 126.746) (width 1) (layer F.Cu) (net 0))
 (segment (start 162.814 132.586) (end 162.7505 130.3655) (width 1) (layer F.Cu) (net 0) (status 10))
 (segment (start 188.6585 116.1415) (end 182.88 116.1415) (width 1) (layer F.Cu) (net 1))
 (segment (start 170.8785 111.0615) (end 177.8 111.0615) (width 1) (layer F.Cu) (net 1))
 (segment (start 177.8 111.0615) (end 182.88 116.1415) (width 1) (layer F.Cu) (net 1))
 (segment (start 170.8785 111.0615) (end 170.8785 106.934) (width 1) (layer F.Cu) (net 1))
 (segment (start 162.814 87.886) (end 162.7505 98.806) (width 1) (layer F.Cu) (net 1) (status 10))
 (segment (start 162.7505 98.806) (end 170.8785 106.934) (width 1) (layer F.Cu) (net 1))
 (segment (start 188.6585 107.2515) (end 196.9135 98.9965) (width 1) (layer F.Cu) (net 5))
 (segment (start 196.9135 98.9965) (end 196.85 87.886) (width 1) (layer F.Cu) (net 5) (status 20))
 (segment (start 188.6585 113.6015) (end 188.6585 107.2515) (width 1) (layer F.Cu) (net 5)))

